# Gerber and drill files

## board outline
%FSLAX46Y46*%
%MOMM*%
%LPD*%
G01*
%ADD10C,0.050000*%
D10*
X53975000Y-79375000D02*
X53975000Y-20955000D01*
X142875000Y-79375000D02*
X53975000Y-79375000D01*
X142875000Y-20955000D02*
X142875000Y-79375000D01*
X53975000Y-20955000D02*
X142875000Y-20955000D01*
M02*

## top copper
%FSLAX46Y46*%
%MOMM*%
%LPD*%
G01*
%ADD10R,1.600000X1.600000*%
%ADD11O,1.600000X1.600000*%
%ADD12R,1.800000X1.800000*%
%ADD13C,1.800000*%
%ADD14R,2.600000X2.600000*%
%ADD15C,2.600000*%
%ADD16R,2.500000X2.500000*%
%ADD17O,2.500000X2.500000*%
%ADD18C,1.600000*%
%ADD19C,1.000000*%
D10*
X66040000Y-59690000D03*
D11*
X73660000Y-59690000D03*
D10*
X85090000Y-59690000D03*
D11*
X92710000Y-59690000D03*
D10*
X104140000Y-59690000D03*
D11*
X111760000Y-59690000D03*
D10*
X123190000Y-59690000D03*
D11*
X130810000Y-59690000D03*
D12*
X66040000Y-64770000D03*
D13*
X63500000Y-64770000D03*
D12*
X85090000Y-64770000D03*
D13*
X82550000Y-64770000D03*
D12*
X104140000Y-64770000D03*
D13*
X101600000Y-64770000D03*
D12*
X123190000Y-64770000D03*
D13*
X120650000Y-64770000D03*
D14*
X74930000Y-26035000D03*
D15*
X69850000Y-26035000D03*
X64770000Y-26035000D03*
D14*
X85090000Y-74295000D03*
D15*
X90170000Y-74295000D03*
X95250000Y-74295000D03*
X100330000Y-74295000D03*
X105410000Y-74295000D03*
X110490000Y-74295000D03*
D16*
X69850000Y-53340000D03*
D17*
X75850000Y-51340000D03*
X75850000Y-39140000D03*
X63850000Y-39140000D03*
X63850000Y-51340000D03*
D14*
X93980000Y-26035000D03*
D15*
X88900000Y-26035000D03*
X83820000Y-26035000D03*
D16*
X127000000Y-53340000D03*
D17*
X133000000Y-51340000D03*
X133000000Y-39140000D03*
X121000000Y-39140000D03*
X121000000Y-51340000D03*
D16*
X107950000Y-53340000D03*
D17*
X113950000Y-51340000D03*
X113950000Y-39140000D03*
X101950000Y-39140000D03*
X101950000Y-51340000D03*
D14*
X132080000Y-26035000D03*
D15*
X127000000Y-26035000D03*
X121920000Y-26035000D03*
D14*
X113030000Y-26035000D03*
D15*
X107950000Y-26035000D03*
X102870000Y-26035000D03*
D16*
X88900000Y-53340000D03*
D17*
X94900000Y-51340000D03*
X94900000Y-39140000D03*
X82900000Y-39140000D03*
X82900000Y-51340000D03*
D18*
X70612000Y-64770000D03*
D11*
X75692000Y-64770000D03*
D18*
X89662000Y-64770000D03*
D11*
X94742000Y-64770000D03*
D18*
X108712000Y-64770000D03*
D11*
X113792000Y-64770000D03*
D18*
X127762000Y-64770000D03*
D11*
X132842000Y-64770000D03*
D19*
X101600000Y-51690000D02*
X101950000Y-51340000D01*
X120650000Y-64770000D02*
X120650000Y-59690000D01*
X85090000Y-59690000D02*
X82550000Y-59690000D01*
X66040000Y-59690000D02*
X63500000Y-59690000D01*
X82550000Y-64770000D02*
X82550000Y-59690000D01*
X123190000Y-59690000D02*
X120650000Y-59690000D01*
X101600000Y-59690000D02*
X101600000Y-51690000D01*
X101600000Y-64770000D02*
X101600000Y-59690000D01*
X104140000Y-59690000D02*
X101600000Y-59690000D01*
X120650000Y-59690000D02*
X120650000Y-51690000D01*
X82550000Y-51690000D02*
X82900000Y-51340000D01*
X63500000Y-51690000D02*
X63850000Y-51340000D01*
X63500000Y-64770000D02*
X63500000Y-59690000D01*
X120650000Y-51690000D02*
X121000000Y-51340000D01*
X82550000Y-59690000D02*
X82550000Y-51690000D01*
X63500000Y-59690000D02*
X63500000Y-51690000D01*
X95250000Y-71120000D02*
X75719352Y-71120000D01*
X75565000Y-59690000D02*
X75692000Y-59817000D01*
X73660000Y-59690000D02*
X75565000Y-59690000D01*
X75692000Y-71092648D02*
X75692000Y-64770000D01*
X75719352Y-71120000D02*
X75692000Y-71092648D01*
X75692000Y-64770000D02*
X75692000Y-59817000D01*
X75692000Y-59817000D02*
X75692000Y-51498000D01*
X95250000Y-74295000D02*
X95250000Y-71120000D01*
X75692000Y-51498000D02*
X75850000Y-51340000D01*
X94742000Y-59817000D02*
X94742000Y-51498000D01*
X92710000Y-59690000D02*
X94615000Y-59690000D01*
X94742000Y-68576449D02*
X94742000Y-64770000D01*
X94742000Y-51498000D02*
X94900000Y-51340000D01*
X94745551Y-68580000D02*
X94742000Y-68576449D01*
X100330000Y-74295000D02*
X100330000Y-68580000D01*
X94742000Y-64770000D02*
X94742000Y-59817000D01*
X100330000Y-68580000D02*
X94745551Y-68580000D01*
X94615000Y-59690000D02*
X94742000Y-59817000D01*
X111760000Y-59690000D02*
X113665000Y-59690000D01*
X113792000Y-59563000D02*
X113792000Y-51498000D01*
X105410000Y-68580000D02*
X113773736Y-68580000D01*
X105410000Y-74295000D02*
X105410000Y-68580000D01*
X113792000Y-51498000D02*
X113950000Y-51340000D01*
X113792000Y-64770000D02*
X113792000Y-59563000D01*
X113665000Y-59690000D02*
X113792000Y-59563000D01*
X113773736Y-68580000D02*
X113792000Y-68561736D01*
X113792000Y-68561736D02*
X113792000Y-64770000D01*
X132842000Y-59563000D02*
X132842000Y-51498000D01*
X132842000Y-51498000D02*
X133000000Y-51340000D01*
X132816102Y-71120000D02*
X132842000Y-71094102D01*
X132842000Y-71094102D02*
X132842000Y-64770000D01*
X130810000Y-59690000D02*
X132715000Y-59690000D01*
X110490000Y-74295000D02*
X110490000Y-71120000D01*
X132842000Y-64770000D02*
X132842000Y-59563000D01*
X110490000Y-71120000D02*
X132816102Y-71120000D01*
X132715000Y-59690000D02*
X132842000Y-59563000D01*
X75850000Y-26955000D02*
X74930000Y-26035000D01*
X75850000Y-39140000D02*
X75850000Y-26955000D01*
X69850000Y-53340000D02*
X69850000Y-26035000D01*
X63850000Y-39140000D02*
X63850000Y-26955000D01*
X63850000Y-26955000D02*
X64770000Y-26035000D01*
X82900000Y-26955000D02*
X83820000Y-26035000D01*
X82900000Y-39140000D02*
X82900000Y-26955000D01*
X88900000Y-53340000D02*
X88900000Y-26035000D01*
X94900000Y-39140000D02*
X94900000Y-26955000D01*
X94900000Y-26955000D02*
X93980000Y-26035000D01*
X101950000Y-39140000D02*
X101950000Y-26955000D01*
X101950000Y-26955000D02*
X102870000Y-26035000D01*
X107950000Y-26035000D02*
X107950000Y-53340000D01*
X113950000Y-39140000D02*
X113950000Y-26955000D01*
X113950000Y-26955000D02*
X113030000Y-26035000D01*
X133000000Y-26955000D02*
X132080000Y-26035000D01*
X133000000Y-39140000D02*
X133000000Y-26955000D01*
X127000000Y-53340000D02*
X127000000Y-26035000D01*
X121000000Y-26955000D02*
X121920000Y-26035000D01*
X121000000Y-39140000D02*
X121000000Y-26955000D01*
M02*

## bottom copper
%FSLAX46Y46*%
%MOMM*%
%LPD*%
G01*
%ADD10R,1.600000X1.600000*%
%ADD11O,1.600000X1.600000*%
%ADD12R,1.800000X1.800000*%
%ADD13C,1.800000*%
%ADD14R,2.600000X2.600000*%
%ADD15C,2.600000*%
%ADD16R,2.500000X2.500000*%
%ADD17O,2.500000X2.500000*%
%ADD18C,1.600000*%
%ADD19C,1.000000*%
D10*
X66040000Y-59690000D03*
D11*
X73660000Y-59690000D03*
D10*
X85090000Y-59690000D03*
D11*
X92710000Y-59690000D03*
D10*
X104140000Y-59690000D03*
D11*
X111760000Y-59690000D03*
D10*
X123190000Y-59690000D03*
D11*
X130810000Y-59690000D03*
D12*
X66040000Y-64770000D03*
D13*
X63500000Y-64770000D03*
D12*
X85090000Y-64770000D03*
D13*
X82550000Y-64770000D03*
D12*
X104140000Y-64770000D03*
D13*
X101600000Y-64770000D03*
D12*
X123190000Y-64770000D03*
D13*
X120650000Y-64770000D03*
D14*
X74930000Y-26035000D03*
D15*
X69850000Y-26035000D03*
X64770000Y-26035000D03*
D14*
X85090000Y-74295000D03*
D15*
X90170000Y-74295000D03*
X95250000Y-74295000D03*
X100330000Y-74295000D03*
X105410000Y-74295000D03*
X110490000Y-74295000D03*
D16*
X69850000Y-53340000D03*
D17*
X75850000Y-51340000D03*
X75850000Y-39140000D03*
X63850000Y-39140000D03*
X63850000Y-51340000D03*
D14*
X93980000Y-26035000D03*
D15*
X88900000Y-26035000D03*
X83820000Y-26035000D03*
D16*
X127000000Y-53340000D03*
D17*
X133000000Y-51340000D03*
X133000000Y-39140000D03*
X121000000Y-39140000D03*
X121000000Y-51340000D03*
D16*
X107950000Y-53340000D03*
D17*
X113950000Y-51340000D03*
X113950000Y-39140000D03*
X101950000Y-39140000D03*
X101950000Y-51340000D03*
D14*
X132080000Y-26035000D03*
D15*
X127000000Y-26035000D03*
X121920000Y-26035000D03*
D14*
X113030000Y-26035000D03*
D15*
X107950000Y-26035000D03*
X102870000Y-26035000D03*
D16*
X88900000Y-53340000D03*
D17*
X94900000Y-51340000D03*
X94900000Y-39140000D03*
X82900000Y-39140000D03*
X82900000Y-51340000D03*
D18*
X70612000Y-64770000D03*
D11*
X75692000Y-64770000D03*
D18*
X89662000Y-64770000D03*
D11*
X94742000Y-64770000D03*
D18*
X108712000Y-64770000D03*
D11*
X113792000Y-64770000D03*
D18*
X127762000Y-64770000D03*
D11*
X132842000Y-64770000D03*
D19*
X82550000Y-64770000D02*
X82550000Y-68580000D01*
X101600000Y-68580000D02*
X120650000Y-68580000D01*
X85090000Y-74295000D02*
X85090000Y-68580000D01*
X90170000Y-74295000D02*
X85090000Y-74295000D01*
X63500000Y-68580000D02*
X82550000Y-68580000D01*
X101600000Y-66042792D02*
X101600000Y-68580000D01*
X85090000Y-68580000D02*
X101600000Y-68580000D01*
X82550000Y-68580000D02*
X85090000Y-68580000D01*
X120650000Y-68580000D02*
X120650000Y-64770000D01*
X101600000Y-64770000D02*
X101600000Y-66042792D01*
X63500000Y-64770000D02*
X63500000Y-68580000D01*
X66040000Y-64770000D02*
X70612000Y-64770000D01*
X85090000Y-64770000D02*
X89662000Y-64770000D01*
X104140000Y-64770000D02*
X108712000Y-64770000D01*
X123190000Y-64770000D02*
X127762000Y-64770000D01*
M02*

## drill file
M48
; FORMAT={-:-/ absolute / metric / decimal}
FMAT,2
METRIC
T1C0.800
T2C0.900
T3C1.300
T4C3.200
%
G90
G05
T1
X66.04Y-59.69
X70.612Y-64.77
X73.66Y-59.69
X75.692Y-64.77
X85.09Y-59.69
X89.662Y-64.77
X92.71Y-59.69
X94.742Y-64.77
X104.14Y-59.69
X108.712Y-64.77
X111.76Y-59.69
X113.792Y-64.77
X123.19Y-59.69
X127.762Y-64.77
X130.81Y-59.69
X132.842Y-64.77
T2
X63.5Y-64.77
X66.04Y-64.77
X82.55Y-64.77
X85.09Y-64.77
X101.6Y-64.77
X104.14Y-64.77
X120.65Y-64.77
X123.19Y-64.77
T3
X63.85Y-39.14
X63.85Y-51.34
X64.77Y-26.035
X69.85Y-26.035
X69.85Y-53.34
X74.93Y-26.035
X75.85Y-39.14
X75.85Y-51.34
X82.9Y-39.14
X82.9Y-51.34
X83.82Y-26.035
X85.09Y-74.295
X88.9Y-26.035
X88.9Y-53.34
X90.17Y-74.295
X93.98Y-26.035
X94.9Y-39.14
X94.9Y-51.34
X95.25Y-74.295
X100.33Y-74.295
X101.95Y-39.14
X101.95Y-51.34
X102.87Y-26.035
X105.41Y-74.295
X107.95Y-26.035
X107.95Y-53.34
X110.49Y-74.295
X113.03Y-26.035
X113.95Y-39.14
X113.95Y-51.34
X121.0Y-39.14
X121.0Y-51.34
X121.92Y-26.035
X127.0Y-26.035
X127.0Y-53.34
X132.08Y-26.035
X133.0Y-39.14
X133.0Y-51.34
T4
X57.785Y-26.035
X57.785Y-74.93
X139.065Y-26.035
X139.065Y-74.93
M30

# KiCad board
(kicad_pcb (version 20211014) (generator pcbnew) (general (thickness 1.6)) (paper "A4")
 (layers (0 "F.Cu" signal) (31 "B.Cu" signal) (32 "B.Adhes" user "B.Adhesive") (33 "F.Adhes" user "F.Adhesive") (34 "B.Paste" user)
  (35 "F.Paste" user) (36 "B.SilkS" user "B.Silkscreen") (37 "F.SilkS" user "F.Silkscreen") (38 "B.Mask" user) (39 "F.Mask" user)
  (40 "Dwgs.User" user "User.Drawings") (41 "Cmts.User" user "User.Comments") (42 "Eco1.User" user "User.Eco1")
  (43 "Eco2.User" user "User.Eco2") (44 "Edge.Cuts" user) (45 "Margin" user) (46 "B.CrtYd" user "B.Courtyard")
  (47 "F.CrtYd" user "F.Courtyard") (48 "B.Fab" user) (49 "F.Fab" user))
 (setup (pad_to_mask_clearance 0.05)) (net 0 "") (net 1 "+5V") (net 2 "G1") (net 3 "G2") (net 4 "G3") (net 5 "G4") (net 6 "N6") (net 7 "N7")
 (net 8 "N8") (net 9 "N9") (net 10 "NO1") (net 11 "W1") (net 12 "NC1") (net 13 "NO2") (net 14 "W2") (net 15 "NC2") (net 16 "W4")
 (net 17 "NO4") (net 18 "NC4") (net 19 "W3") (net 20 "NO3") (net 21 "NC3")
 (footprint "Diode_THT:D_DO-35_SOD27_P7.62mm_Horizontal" (layer "F.Cu") (at 66.04 59.69)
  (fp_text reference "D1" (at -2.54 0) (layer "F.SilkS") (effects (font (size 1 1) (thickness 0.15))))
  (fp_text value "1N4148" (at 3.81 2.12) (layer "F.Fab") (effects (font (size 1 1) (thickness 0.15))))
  (pad "1" thru_hole rect locked (at 0 0) (size 1.6 1.6) (drill 0.8) (layers *.Cu *.Mask) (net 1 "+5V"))
  (pad "2" thru_hole oval locked (at 7.62 0) (size 1.6 1.6) (drill 0.8) (layers *.Cu *.Mask) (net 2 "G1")))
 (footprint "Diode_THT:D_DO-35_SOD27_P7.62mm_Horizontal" (layer "F.Cu") (at 85.09 59.69)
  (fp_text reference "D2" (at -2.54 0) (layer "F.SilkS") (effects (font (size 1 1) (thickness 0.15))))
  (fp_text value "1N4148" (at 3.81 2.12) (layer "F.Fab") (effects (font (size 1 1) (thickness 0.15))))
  (pad "1" thru_hole rect locked (at 0 0) (size 1.6 1.6) (drill 0.8) (layers *.Cu *.Mask) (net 1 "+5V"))
  (pad "2" thru_hole oval locked (at 7.62 0) (size 1.6 1.6) (drill 0.8) (layers *.Cu *.Mask) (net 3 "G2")))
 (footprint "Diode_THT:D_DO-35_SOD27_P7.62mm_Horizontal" (layer "F.Cu") (at 104.14 59.69)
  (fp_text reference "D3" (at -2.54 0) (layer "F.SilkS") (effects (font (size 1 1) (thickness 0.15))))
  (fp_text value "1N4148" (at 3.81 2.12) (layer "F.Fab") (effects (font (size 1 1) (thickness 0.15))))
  (pad "1" thru_hole rect locked (at 0 0) (size 1.6 1.6) (drill 0.8) (layers *.Cu *.Mask) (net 1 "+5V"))
  (pad "2" thru_hole oval locked (at 7.62 0) (size 1.6 1.6) (drill 0.8) (layers *.Cu *.Mask) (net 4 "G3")))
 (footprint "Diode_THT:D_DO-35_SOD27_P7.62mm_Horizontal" (layer "F.Cu") (at 123.19 59.69)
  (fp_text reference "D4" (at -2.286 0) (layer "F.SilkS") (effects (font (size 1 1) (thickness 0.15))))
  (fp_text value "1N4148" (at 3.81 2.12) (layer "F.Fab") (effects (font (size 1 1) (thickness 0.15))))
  (pad "1" thru_hole rect locked (at 0 0) (size 1.6 1.6) (drill 0.8) (layers *.Cu *.Mask) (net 1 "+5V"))
  (pad "2" thru_hole oval locked (at 7.62 0) (size 1.6 1.6) (drill 0.8) (layers *.Cu *.Mask) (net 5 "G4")))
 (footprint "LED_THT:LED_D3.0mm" (layer "F.Cu") (at 66.04 64.77 180)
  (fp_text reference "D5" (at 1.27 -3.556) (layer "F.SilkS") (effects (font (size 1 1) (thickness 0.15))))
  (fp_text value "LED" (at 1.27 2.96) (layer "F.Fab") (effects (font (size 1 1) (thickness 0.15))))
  (pad "1" thru_hole rect locked (at 0 0 180) (size 1.8 1.8) (drill 0.9) (layers *.Cu *.Mask) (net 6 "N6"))
  (pad "2" thru_hole circle locked (at 2.54 0 180) (size 1.8 1.8) (drill 0.9) (layers *.Cu *.Mask) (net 1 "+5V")))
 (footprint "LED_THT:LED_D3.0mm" (layer "F.Cu") (at 85.09 64.77 180)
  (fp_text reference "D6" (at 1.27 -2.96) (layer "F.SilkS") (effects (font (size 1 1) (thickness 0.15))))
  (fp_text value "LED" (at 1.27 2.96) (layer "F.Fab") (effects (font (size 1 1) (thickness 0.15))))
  (pad "1" thru_hole rect locked (at 0 0 180) (size 1.8 1.8) (drill 0.9) (layers *.Cu *.Mask) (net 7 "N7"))
  (pad "2" thru_hole circle locked (at 2.54 0 180) (size 1.8 1.8) (drill 0.9) (layers *.Cu *.Mask) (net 1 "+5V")))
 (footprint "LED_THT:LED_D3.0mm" (layer "F.Cu") (at 104.14 64.77 180)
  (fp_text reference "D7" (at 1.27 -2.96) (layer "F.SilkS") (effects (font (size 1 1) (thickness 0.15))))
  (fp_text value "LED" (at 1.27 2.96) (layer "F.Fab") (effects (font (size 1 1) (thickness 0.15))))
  (pad "1" thru_hole rect locked (at 0 0 180) (size 1.8 1.8) (drill 0.9) (layers *.Cu *.Mask) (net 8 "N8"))
  (pad "2" thru_hole circle locked (at 2.54 0 180) (size 1.8 1.8) (drill 0.9) (layers *.Cu *.Mask) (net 1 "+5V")))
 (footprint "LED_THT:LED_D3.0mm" (layer "F.Cu") (at 123.19 64.77 180)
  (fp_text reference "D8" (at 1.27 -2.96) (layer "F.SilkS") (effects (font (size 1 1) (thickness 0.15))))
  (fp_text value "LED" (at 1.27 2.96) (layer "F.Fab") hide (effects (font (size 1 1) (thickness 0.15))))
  (pad "1" thru_hole rect locked (at 0 0 180) (size 1.8 1.8) (drill 0.9) (layers *.Cu *.Mask) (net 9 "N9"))
  (pad "2" thru_hole circle locked (at 2.54 0 180) (size 1.8 1.8) (drill 0.9) (layers *.Cu *.Mask) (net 1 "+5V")))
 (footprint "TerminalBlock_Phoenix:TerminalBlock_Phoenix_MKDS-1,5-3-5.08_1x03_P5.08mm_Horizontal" (layer "F.Cu") (at 74.93 26.035 180)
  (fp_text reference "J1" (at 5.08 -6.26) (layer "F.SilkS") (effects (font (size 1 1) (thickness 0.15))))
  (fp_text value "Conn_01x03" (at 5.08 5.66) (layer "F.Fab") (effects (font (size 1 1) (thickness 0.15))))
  (pad "1" thru_hole rect locked (at 0 0 180) (size 2.6 2.6) (drill 1.3) (layers *.Cu *.Mask) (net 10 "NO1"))
  (pad "2" thru_hole circle locked (at 5.08 0 180) (size 2.6 2.6) (drill 1.3) (layers *.Cu *.Mask) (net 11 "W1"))
  (pad "3" thru_hole circle locked (at 10.16 0 180) (size 2.6 2.6) (drill 1.3) (layers *.Cu *.Mask) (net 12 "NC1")))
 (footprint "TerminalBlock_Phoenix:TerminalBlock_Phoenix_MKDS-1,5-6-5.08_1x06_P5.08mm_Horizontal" (layer "F.Cu") (at 85.09 74.295)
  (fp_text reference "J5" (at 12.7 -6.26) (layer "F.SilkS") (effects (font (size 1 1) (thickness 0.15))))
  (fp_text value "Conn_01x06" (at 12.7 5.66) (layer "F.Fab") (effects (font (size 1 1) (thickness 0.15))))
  (pad "1" thru_hole rect locked (at 0 0) (size 2.6 2.6) (drill 1.3) (layers *.Cu *.Mask) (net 1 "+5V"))
  (pad "2" thru_hole circle locked (at 5.08 0) (size 2.6 2.6) (drill 1.3) (layers *.Cu *.Mask) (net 1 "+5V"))
  (pad "3" thru_hole circle locked (at 10.16 0) (size 2.6 2.6) (drill 1.3) (layers *.Cu *.Mask) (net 2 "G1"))
  (pad "4" thru_hole circle locked (at 15.24 0) (size 2.6 2.6) (drill 1.3) (layers *.Cu *.Mask) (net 3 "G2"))
  (pad "5" thru_hole circle locked (at 20.32 0) (size 2.6 2.6) (drill 1.3) (layers *.Cu *.Mask) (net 4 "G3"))
  (pad "6" thru_hole circle locked (at 25.4 0) (size 2.6 2.6) (drill 1.3) (layers *.Cu *.Mask) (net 5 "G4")))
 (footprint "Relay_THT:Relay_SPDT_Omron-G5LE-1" (layer "F.Cu") (at 69.85 53.34 180)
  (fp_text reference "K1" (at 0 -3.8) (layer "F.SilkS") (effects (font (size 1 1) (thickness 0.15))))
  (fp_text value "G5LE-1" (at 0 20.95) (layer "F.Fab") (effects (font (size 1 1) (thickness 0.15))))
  (pad "1" thru_hole rect locked (at 0 0 180) (size 2.5 2.5) (drill 1.3) (layers *.Cu *.Mask) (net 11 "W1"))
  (pad "2" thru_hole oval locked (at -6 2 180) (size 2.5 2.5) (drill 1.3) (layers *.Cu *.Mask) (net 2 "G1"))
  (pad "3" thru_hole oval locked (at -6 14.2 180) (size 2.5 2.5) (drill 1.3) (layers *.Cu *.Mask) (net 10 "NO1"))
  (pad "4" thru_hole oval locked (at 6 14.2 180) (size 2.5 2.5) (drill 1.3) (layers *.Cu *.Mask) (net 12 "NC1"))
  (pad "5" thru_hole oval locked (at 6 2 180) (size 2.5 2.5) (drill 1.3) (layers *.Cu *.Mask) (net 1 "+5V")))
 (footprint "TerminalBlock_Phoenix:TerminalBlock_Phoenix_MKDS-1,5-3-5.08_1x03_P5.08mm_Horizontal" (layer "F.Cu") (at 93.98 26.035 180)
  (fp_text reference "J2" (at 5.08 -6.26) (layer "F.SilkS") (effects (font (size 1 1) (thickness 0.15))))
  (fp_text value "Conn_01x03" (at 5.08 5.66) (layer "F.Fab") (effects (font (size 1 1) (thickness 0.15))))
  (pad "1" thru_hole rect locked (at 0 0 180) (size 2.6 2.6) (drill 1.3) (layers *.Cu *.Mask) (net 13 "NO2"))
  (pad "2" thru_hole circle locked (at 5.08 0 180) (size 2.6 2.6) (drill 1.3) (layers *.Cu *.Mask) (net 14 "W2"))
  (pad "3" thru_hole circle locked (at 10.16 0 180) (size 2.6 2.6) (drill 1.3) (layers *.Cu *.Mask) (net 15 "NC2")))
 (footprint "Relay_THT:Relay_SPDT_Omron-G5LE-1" (layer "F.Cu") (at 127 53.34 180)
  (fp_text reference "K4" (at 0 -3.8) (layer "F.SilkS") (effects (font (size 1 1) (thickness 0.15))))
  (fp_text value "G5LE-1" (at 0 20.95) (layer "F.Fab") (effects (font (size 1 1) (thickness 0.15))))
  (pad "1" thru_hole rect locked (at 0 0 180) (size 2.5 2.5) (drill 1.3) (layers *.Cu *.Mask) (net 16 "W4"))
  (pad "2" thru_hole oval locked (at -6 2 180) (size 2.5 2.5) (drill 1.3) (layers *.Cu *.Mask) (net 5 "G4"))
  (pad "3" thru_hole oval locked (at -6 14.2 180) (size 2.5 2.5) (drill 1.3) (layers *.Cu *.Mask) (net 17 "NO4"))
  (pad "4" thru_hole oval locked (at 6 14.2 180) (size 2.5 2.5) (drill 1.3) (layers *.Cu *.Mask) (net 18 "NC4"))
  (pad "5" thru_hole oval locked (at 6 2 180) (size 2.5 2.5) (drill 1.3) (layers *.Cu *.Mask) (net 1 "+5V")))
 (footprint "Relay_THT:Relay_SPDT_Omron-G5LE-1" (layer "F.Cu") (at 107.95 53.34 180)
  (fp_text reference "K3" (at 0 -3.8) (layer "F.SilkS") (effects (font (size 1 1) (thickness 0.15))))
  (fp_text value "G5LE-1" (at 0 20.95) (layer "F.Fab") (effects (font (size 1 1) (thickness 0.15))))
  (pad "1" thru_hole rect locked (at 0 0 180) (size 2.5 2.5) (drill 1.3) (layers *.Cu *.Mask) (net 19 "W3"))
  (pad "2" thru_hole oval locked (at -6 2 180) (size 2.5 2.5) (drill 1.3) (layers *.Cu *.Mask) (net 4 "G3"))
  (pad "3" thru_hole oval locked (at -6 14.2 180) (size 2.5 2.5) (drill 1.3) (layers *.Cu *.Mask) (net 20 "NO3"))
  (pad "4" thru_hole oval locked (at 6 14.2 180) (size 2.5 2.5) (drill 1.3) (layers *.Cu *.Mask) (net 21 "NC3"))
  (pad "5" thru_hole oval locked (at 6 2 180) (size 2.5 2.5) (drill 1.3) (layers *.Cu *.Mask) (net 1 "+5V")))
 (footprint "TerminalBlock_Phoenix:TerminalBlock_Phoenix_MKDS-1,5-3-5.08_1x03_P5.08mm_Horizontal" (layer "F.Cu") (at 132.08 26.035 180)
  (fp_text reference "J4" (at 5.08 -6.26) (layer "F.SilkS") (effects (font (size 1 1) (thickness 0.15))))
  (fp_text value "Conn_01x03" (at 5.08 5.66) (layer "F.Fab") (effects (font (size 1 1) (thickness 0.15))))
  (pad "1" thru_hole rect locked (at 0 0 180) (size 2.6 2.6) (drill 1.3) (layers *.Cu *.Mask) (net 17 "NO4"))
  (pad "2" thru_hole circle locked (at 5.08 0 180) (size 2.6 2.6) (drill 1.3) (layers *.Cu *.Mask) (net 16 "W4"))
  (pad "3" thru_hole circle locked (at 10.16 0 180) (size 2.6 2.6) (drill 1.3) (layers *.Cu *.Mask) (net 18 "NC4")))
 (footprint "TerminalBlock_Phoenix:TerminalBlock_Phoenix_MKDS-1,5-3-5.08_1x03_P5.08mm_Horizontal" (layer "F.Cu") (at 113.03 26.035 180)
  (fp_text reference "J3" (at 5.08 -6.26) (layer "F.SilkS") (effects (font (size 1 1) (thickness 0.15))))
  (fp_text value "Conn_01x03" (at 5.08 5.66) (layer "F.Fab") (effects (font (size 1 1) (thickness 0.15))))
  (pad "1" thru_hole rect locked (at 0 0 180) (size 2.6 2.6) (drill 1.3) (layers *.Cu *.Mask) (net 20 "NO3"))
  (pad "2" thru_hole circle locked (at 5.08 0 180) (size 2.6 2.6) (drill 1.3) (layers *.Cu *.Mask) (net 19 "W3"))
  (pad "3" thru_hole circle locked (at 10.16 0 180) (size 2.6 2.6) (drill 1.3) (layers *.Cu *.Mask) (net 21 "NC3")))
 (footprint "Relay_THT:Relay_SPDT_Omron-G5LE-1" (layer "F.Cu") (at 88.9 53.34 180)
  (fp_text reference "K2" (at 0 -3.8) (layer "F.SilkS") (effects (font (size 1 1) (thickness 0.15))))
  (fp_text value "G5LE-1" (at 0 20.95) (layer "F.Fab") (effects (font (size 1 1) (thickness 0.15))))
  (pad "1" thru_hole rect locked (at 0 0 180) (size 2.5 2.5) (drill 1.3) (layers *.Cu *.Mask) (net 14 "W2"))
  (pad "2" thru_hole oval locked (at -6 2 180) (size 2.5 2.5) (drill 1.3) (layers *.Cu *.Mask) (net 3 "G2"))
  (pad "3" thru_hole oval locked (at -6 14.2 180) (size 2.5 2.5) (drill 1.3) (layers *.Cu *.Mask) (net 13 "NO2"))
  (pad "4" thru_hole oval locked (at 6 14.2 180) (size 2.5 2.5) (drill 1.3) (layers *.Cu *.Mask) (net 15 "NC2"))
  (pad "5" thru_hole oval locked (at 6 2 180) (size 2.5 2.5) (drill 1.3) (layers *.Cu *.Mask) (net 1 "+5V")))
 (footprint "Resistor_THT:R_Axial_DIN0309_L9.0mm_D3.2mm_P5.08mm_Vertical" (layer "F.Cu") (at 70.612 64.77)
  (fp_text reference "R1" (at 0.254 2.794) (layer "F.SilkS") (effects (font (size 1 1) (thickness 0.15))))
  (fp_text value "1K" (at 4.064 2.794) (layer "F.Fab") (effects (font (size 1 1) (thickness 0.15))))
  (pad "1" thru_hole circle locked (at 0 0) (size 1.6 1.6) (drill 0.8) (layers *.Cu *.Mask) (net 6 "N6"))
  (pad "2" thru_hole oval locked (at 5.08 0) (size 1.6 1.6) (drill 0.8) (layers *.Cu *.Mask) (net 2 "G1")))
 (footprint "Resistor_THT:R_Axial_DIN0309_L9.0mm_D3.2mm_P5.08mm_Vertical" (layer "F.Cu") (at 89.662 64.77)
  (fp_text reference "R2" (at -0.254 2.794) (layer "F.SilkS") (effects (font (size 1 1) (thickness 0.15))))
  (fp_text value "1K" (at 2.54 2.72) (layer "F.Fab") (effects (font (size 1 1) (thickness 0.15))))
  (pad "1" thru_hole circle locked (at 0 0) (size 1.6 1.6) (drill 0.8) (layers *.Cu *.Mask) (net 7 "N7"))
  (pad "2" thru_hole oval locked (at 5.08 0) (size 1.6 1.6) (drill 0.8) (layers *.Cu *.Mask) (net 3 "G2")))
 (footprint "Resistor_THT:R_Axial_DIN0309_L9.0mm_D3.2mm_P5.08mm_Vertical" (layer "F.Cu") (at 108.712 64.77)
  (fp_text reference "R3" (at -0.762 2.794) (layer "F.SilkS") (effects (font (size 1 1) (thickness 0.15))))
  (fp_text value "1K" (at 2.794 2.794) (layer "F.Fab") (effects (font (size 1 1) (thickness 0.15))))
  (pad "1" thru_hole circle locked (at 0 0) (size 1.6 1.6) (drill 0.8) (layers *.Cu *.Mask) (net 8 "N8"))
  (pad "2" thru_hole oval locked (at 5.08 0) (size 1.6 1.6) (drill 0.8) (layers *.Cu *.Mask) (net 4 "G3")))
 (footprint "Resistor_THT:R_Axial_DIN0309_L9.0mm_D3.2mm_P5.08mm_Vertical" (layer "F.Cu") (at 127.762 64.77)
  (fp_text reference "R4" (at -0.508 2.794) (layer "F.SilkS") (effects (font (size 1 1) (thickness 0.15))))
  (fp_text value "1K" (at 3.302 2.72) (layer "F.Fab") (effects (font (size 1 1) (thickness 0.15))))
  (pad "1" thru_hole circle locked (at 0 0) (size 1.6 1.6) (drill 0.8) (layers *.Cu *.Mask) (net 9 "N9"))
  (pad "2" thru_hole oval locked (at 5.08 0) (size 1.6 1.6) (drill 0.8) (layers *.Cu *.Mask) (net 5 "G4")))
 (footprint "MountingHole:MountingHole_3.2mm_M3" (layer "F.Cu") (at 139.065 26.035)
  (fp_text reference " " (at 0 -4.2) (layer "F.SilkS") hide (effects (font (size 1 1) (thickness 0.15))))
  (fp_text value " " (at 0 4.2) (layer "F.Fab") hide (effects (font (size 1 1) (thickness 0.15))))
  (pad "" np_thru_hole circle locked (at 0 0) (size 3.2 3.2) (drill 3.2) (layers *.Cu *.Mask)))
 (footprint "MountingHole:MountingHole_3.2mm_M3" (layer "F.Cu") (at 139.065 74.93)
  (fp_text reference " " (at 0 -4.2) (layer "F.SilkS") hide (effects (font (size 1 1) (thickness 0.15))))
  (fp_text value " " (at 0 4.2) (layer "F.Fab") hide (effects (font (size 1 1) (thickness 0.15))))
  (pad "" np_thru_hole circle locked (at 0 0) (size 3.2 3.2) (drill 3.2) (layers *.Cu *.Mask)))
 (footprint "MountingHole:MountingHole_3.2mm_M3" (layer "F.Cu") (at 57.785 26.035)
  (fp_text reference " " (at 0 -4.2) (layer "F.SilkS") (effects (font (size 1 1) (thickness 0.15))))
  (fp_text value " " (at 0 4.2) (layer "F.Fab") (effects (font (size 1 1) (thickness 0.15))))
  (pad "" np_thru_hole circle locked (at 0 0) (size 3.2 3.2) (drill 3.2) (layers *.Cu *.Mask)))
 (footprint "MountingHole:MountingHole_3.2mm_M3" (layer "F.Cu") (at 57.785 74.93)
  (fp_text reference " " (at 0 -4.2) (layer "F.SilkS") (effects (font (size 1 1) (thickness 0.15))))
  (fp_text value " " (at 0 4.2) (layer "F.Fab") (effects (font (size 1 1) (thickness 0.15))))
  (pad "" np_thru_hole circle locked (at 0 0) (size 3.2 3.2) (drill 3.2) (layers *.Cu *.Mask)))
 (gr_line (start 53.975 79.375) (end 53.975 20.955) (layer "Edge.Cuts") (width 0.05))
 (gr_line (start 142.875 79.375) (end 53.975 79.375) (layer "Edge.Cuts") (width 0.05))
 (gr_line (start 142.875 20.955) (end 142.875 79.375) (layer "Edge.Cuts") (width 0.05))
 (gr_line (start 53.975 20.955) (end 142.875 20.955) (layer "Edge.Cuts") (width 0.05))
 (segment (start 101.6 51.69) (end 101.95 51.34) (width 1) (layer "F.Cu") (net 1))
 (segment (start 120.65 64.77) (end 120.65 59.69) (width 1) (layer "F.Cu") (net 1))
 (segment (start 85.09 59.69) (end 82.55 59.69) (width 1) (layer "F.Cu") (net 1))
 (segment (start 66.04 59.69) (end 63.5 59.69) (width 1) (layer "F.Cu") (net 1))
 (segment (start 82.55 64.77) (end 82.55 59.69) (width 1) (layer "F.Cu") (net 1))
 (segment (start 123.19 59.69) (end 120.65 59.69) (width 1) (layer "F.Cu") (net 1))
 (segment (start 101.6 59.69) (end 101.6 51.69) (width 1) (layer "F.Cu") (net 1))
 (segment (start 101.6 64.77) (end 101.6 59.69) (width 1) (layer "F.Cu") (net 1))
 (segment (start 104.14 59.69) (end 101.6 59.69) (width 1) (layer "F.Cu") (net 1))
 (segment (start 120.65 59.69) (end 120.65 51.69) (width 1) (layer "F.Cu") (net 1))
 (segment (start 82.55 51.69) (end 82.9 51.34) (width 1) (layer "F.Cu") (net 1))
 (segment (start 63.5 51.69) (end 63.85 51.34) (width 1) (layer "F.Cu") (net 1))
 (segment (start 63.5 64.77) (end 63.5 59.69) (width 1) (layer "F.Cu") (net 1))
 (segment (start 120.65 51.69) (end 121 51.34) (width 1) (layer "F.Cu") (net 1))
 (segment (start 82.55 59.69) (end 82.55 51.69) (width 1) (layer "F.Cu") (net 1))
 (segment (start 63.5 59.69) (end 63.5 51.69) (width 1) (layer "F.Cu") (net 1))
 (segment (start 82.55 64.77) (end 82.55 68.58) (width 1) (layer "B.Cu") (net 1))
 (segment (start 101.6 68.58) (end 120.65 68.58) (width 1) (layer "B.Cu") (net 1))
 (segment (start 85.09 74.295) (end 85.09 68.58) (width 1) (layer "B.Cu") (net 1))
 (segment (start 90.17 74.295) (end 85.09 74.295) (width 1) (layer "B.Cu") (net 1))
 (segment (start 63.5 68.58) (end 82.55 68.58) (width 1) (layer "B.Cu") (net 1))
 (segment (start 101.6 66.042792) (end 101.6 68.58) (width 1) (layer "B.Cu") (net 1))
 (segment (start 85.09 68.58) (end 101.6 68.58) (width 1) (layer "B.Cu") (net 1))
 (segment (start 82.55 68.58) (end 85.09 68.58) (width 1) (layer "B.Cu") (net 1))
 (segment (start 120.65 68.58) (end 120.65 64.77) (width 1) (layer "B.Cu") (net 1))
 (segment (start 101.6 64.77) (end 101.6 66.042792) (width 1) (layer "B.Cu") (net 1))
 (segment (start 63.5 64.77) (end 63.5 68.58) (width 1) (layer "B.Cu") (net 1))
 (segment (start 95.25 71.12) (end 75.719352 71.12) (width 1) (layer "F.Cu") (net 2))
 (segment (start 75.565 59.69) (end 75.692 59.817) (width 1) (layer "F.Cu") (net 2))
 (segment (start 73.66 59.69) (end 75.565 59.69) (width 1) (layer "F.Cu") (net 2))
 (segment (start 75.692 71.092648) (end 75.692 64.77) (width 1) (layer "F.Cu") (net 2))
 (segment (start 75.719352 71.12) (end 75.692 71.092648) (width 1) (layer "F.Cu") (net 2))
 (segment (start 75.692 64.77) (end 75.692 59.817) (width 1) (layer "F.Cu") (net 2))
 (segment (start 75.692 59.817) (end 75.692 51.498) (width 1) (layer "F.Cu") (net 2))
 (segment (start 95.25 74.295) (end 95.25 71.12) (width 1) (layer "F.Cu") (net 2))
 (segment (start 75.692 51.498) (end 75.85 51.34) (width 1) (layer "F.Cu") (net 2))
 (segment (start 94.742 59.817) (end 94.742 51.498) (width 1) (layer "F.Cu") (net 3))
 (segment (start 92.71 59.69) (end 94.615 59.69) (width 1) (layer "F.Cu") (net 3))
 (segment (start 94.742 68.576449) (end 94.742 64.77) (width 1) (layer "F.Cu") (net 3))
 (segment (start 94.742 51.498) (end 94.9 51.34) (width 1) (layer "F.Cu") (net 3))
 (segment (start 94.745551 68.58) (end 94.742 68.576449) (width 1) (layer "F.Cu") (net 3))
 (segment (start 100.33 74.295) (end 100.33 68.58) (width 1) (layer "F.Cu") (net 3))
 (segment (start 94.742 64.77) (end 94.742 59.817) (width 1) (layer "F.Cu") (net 3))
 (segment (start 100.33 68.58) (end 94.745551 68.58) (width 1) (layer "F.Cu") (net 3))
 (segment (start 94.615 59.69) (end 94.742 59.817) (width 1) (layer "F.Cu") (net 3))
 (segment (start 111.76 59.69) (end 113.665 59.69) (width 1) (layer "F.Cu") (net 4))
 (segment (start 113.792 59.563) (end 113.792 51.498) (width 1) (layer "F.Cu") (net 4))
 (segment (start 105.41 68.58) (end 113.773736 68.58) (width 1) (layer "F.Cu") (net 4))
 (segment (start 105.41 74.295) (end 105.41 68.58) (width 1) (layer "F.Cu") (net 4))
 (segment (start 113.792 51.498) (end 113.95 51.34) (width 1) (layer "F.Cu") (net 4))
 (segment (start 113.792 64.77) (end 113.792 59.563) (width 1) (layer "F.Cu") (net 4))
 (segment (start 113.665 59.69) (end 113.792 59.563) (width 1) (layer "F.Cu") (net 4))
 (segment (start 113.773736 68.58) (end 113.792 68.561736) (width 1) (layer "F.Cu") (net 4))
 (segment (start 113.792 68.561736) (end 113.792 64.77) (width 1) (layer "F.Cu") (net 4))
 (segment (start 132.842 59.563) (end 132.842 51.498) (width 1) (layer "F.Cu") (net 5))
 (segment (start 132.842 51.498) (end 133 51.34) (width 1) (layer "F.Cu") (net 5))
 (segment (start 132.816102 71.12) (end 132.842 71.094102) (width 1) (layer "F.Cu") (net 5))
 (segment (start 132.842 71.094102) (end 132.842 64.77) (width 1) (layer "F.Cu") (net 5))
 (segment (start 130.81 59.69) (end 132.715 59.69) (width 1) (layer "F.Cu") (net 5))
 (segment (start 110.49 74.295) (end 110.49 71.12) (width 1) (layer "F.Cu") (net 5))
 (segment (start 132.842 64.77) (end 132.842 59.563) (width 1) (layer "F.Cu") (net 5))
 (segment (start 110.49 71.12) (end 132.816102 71.12) (width 1) (layer "F.Cu") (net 5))
 (segment (start 132.715 59.69) (end 132.842 59.563) (width 1) (layer "F.Cu") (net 5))
 (segment (start 66.04 64.77) (end 70.612 64.77) (width 1) (layer "B.Cu") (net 6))
 (segment (start 85.09 64.77) (end 89.662 64.77) (width 1) (layer "B.Cu") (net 7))
 (segment (start 104.14 64.77) (end 108.712 64.77) (width 1) (layer "B.Cu") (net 8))
 (segment (start 123.19 64.77) (end 127.762 64.77) (width 1) (layer "B.Cu") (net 9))
 (segment (start 75.85 26.955) (end 74.93 26.035) (width 1) (layer "F.Cu") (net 10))
 (segment (start 75.85 39.14) (end 75.85 26.955) (width 1) (layer "F.Cu") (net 10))
 (segment (start 69.85 53.34) (end 69.85 26.035) (width 1) (layer "F.Cu") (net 11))
 (segment (start 63.85 39.14) (end 63.85 26.955) (width 1) (layer "F.Cu") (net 12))
 (segment (start 63.85 26.955) (end 64.77 26.035) (width 1) (layer "F.Cu") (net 12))
 (segment (start 82.9 26.955) (end 83.82 26.035) (width 1) (layer "F.Cu") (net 15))
 (segment (start 82.9 39.14) (end 82.9 26.955) (width 1) (layer "F.Cu") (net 15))
 (segment (start 88.9 53.34) (end 88.9 26.035) (width 1) (layer "F.Cu") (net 14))
 (segment (start 94.9 39.14) (end 94.9 26.955) (width 1) (layer "F.Cu") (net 13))
 (segment (start 94.9 26.955) (end 93.98 26.035) (width 1) (layer "F.Cu") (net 13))
 (segment (start 101.95 39.14) (end 101.95 26.955) (width 1) (layer "F.Cu") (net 21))
 (segment (start 101.95 26.955) (end 102.87 26.035) (width 1) (layer "F.Cu") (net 21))
 (segment (start 107.95 26.035) (end 107.95 53.34) (width 1) (layer "F.Cu") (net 19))
 (segment (start 113.95 39.14) (end 113.95 26.955) (width 1) (layer "F.Cu") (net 20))
 (segment (start 113.95 26.955) (end 113.03 26.035) (width 1) (layer "F.Cu") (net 20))
 (segment (start 133 26.955) (end 132.08 26.035) (width 1) (layer "F.Cu") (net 17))
 (segment (start 133 39.14) (end 133 26.955) (width 1) (layer "F.Cu") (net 17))
 (segment (start 127 53.34) (end 127 26.035) (width 1) (layer "F.Cu") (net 16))
 (segment (start 121 26.955) (end 121.92 26.035) (width 1) (layer "F.Cu") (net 18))
 (segment (start 121 39.14) (end 121 26.955) (width 1) (layer "F.Cu") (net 18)))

